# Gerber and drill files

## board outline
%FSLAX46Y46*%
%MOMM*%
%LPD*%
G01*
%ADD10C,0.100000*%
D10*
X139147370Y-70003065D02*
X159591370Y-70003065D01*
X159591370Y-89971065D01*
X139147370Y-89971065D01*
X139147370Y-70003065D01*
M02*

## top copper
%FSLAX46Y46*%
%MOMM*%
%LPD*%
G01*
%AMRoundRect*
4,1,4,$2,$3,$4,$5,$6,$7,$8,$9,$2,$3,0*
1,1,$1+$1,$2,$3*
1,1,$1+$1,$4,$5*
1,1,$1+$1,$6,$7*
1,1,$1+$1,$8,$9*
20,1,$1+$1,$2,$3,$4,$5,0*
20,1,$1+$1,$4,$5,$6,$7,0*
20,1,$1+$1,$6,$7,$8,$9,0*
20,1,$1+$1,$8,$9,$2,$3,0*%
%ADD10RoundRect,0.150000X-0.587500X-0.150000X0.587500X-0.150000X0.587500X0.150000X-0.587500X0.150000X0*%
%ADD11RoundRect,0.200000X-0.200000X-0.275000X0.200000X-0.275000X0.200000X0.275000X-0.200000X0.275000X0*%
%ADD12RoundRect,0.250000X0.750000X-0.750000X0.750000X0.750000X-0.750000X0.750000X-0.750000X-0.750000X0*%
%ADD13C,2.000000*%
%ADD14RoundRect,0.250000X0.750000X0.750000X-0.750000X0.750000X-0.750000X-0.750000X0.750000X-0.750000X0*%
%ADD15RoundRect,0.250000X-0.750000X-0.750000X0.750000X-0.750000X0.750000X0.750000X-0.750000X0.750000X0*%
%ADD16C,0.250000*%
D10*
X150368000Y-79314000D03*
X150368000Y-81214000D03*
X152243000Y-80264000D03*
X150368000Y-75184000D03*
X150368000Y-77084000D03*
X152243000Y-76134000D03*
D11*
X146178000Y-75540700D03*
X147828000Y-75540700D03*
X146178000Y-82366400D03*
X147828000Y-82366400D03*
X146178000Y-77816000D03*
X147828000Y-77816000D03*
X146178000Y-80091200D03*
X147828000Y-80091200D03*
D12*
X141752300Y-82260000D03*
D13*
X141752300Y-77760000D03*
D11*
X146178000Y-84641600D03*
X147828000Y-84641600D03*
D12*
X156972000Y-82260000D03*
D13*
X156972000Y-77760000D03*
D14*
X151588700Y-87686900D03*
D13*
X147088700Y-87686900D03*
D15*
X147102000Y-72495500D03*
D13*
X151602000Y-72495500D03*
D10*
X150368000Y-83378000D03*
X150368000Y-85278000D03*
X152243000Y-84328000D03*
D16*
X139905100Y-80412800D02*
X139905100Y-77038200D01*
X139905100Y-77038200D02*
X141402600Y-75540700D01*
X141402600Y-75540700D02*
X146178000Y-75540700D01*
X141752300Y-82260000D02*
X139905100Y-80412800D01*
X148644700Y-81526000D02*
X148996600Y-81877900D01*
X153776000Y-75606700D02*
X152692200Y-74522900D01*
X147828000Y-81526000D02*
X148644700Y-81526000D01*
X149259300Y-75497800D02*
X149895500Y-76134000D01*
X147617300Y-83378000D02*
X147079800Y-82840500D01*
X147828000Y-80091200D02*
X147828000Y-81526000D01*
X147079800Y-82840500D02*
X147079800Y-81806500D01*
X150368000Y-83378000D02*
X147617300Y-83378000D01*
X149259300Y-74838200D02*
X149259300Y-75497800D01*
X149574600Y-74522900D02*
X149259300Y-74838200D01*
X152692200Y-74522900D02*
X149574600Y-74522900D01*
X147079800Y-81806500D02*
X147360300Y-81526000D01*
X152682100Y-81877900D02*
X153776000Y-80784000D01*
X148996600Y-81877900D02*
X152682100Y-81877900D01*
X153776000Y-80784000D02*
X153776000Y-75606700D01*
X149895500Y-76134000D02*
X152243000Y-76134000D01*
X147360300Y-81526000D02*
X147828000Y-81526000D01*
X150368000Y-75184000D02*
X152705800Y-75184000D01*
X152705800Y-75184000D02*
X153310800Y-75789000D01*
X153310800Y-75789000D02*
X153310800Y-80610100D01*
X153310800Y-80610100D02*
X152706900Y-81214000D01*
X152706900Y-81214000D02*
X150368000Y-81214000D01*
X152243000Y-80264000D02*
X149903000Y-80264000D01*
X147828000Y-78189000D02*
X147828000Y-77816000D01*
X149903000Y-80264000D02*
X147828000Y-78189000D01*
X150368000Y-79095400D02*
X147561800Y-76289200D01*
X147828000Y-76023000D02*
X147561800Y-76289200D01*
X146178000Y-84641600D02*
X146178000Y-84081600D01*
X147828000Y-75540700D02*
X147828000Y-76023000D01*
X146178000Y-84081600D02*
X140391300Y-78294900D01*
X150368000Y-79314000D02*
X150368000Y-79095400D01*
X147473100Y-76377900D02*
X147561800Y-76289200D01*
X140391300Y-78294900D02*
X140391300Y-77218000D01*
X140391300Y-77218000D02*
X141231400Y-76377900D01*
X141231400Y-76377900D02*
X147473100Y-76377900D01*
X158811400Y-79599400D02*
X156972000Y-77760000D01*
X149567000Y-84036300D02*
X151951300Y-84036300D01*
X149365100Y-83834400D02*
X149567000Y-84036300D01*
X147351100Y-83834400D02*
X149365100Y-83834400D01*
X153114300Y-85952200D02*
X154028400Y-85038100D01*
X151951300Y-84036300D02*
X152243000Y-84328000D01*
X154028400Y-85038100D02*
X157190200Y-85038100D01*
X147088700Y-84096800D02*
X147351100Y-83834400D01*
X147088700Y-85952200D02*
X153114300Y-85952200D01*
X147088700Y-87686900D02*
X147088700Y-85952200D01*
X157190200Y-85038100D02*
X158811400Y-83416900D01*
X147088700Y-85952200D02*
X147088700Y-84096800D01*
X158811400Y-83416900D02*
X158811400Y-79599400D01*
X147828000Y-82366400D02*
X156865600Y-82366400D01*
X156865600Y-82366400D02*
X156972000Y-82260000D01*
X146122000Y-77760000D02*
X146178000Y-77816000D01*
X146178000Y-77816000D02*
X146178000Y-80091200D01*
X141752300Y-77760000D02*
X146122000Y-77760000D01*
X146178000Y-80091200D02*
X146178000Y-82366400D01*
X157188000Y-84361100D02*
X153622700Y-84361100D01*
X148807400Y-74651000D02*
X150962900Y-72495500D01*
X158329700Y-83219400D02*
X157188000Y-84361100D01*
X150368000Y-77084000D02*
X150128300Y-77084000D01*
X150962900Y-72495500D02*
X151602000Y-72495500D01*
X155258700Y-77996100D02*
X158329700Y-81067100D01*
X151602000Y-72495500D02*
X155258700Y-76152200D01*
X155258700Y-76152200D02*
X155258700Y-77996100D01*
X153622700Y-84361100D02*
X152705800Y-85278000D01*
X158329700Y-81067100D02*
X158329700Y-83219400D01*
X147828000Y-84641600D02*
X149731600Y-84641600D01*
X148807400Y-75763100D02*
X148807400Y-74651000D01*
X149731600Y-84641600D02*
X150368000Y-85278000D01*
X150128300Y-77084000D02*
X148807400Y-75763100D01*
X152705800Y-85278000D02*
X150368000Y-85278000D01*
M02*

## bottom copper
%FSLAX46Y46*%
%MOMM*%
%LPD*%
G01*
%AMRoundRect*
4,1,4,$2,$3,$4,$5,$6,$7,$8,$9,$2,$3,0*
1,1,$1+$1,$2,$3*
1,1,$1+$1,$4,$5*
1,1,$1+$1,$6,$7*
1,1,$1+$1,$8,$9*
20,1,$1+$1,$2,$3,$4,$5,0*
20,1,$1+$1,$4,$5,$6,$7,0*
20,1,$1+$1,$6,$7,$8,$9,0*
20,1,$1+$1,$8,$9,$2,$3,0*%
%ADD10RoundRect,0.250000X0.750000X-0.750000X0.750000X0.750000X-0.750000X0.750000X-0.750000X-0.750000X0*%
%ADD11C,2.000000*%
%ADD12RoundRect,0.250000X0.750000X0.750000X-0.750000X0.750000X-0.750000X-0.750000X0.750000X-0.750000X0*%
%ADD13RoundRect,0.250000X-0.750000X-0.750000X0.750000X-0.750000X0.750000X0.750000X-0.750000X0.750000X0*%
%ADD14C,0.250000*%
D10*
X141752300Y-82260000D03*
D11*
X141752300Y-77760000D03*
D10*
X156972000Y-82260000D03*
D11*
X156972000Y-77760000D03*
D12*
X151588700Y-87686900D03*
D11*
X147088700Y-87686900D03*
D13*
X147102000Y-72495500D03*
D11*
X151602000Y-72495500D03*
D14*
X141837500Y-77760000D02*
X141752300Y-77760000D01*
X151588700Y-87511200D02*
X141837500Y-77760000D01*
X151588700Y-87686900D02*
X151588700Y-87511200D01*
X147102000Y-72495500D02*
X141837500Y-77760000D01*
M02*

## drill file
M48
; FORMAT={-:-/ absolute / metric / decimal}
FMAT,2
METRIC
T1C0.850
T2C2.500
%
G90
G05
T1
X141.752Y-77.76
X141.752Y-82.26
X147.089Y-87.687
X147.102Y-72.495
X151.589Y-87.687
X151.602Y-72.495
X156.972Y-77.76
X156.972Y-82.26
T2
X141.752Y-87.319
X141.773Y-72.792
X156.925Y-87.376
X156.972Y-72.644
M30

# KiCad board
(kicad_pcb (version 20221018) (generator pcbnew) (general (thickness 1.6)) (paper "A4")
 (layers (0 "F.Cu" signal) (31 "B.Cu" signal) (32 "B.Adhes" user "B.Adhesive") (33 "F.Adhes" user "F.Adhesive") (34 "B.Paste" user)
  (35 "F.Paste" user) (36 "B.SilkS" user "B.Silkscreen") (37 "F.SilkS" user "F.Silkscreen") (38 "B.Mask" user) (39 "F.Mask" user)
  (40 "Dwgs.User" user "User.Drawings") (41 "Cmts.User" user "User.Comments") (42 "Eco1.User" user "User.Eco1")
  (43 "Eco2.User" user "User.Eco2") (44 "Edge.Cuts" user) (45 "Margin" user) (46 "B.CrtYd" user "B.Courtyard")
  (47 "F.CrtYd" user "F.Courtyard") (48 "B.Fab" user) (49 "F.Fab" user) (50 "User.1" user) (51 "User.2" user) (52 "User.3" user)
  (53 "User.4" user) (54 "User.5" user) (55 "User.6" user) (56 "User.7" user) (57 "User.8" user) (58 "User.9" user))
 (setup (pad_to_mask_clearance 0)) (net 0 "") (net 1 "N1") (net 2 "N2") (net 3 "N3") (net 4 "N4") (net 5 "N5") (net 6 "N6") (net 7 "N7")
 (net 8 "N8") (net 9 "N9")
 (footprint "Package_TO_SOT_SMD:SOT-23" (layer "F.Cu") (at 151.3055 80.264)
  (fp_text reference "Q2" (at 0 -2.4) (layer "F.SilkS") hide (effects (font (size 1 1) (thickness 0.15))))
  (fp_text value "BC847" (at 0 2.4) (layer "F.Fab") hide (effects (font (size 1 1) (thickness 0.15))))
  (pad "1" smd roundrect (at -0.9375 -0.95) (size 1.475 0.6) (layers "F.Cu" "F.Paste" "F.Mask") (roundrect_rratio 0.25) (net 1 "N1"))
  (pad "2" smd roundrect (at -0.9375 0.95) (size 1.475 0.6) (layers "F.Cu" "F.Paste" "F.Mask") (roundrect_rratio 0.25) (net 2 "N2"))
  (pad "3" smd roundrect (at 0.9375 0) (size 1.475 0.6) (layers "F.Cu" "F.Paste" "F.Mask") (roundrect_rratio 0.25) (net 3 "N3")))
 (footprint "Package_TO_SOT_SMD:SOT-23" (layer "F.Cu") (at 151.3055 76.134)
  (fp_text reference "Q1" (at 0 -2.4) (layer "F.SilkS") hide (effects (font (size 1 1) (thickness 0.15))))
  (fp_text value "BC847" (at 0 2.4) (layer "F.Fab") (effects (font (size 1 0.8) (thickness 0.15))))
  (pad "1" smd roundrect (at -0.9375 -0.95) (size 1.475 0.6) (layers "F.Cu" "F.Paste" "F.Mask") (roundrect_rratio 0.25) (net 2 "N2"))
  (pad "2" smd roundrect (at -0.9375 0.95) (size 1.475 0.6) (layers "F.Cu" "F.Paste" "F.Mask") (roundrect_rratio 0.25) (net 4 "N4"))
  (pad "3" smd roundrect (at 0.9375 0) (size 1.475 0.6) (layers "F.Cu" "F.Paste" "F.Mask") (roundrect_rratio 0.25) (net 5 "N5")))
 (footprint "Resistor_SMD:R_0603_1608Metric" (layer "F.Cu") (at 147.003 75.5407)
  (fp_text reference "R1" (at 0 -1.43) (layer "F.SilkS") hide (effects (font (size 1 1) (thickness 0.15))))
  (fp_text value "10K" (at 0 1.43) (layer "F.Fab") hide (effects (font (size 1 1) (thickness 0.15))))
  (pad "1" smd roundrect (at -0.825 0) (size 0.8 0.95) (layers "F.Cu" "F.Paste" "F.Mask") (roundrect_rratio 0.25) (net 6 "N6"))
  (pad "2" smd roundrect (at 0.825 0) (size 0.8 0.95) (layers "F.Cu" "F.Paste" "F.Mask") (roundrect_rratio 0.25) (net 1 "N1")))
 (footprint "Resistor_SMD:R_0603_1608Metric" (layer "F.Cu") (at 147.003 82.3664)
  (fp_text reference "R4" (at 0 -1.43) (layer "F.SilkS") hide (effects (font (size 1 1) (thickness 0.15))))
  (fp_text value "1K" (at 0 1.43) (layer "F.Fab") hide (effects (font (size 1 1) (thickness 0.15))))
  (pad "1" smd roundrect (at -0.825 0) (size 0.8 0.95) (layers "F.Cu" "F.Paste" "F.Mask") (roundrect_rratio 0.25) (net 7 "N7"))
  (pad "2" smd roundrect (at 0.825 0) (size 0.8 0.95) (layers "F.Cu" "F.Paste" "F.Mask") (roundrect_rratio 0.25) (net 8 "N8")))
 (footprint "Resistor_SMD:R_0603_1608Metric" (layer "F.Cu") (at 147.003 77.816)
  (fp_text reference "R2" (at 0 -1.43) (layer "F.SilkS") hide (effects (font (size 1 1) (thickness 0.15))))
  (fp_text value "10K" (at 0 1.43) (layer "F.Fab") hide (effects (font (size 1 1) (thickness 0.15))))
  (pad "1" smd roundrect (at -0.825 0) (size 0.8 0.95) (layers "F.Cu" "F.Paste" "F.Mask") (roundrect_rratio 0.25) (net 7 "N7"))
  (pad "2" smd roundrect (at 0.825 0) (size 0.8 0.95) (layers "F.Cu" "F.Paste" "F.Mask") (roundrect_rratio 0.25) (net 3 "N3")))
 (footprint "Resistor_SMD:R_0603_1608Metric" (layer "F.Cu") (at 147.003 80.0912)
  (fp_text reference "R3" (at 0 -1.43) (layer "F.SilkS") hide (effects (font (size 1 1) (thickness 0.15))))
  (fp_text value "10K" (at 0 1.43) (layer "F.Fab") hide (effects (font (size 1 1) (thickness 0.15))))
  (pad "1" smd roundrect (at -0.825 0) (size 0.8 0.95) (layers "F.Cu" "F.Paste" "F.Mask") (roundrect_rratio 0.25) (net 7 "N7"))
  (pad "2" smd roundrect (at 0.825 0) (size 0.8 0.95) (layers "F.Cu" "F.Paste" "F.Mask") (roundrect_rratio 0.25) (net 5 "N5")))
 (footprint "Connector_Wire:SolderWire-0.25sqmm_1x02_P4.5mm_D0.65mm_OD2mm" (layer "F.Cu") (at 141.7523 82.26 90)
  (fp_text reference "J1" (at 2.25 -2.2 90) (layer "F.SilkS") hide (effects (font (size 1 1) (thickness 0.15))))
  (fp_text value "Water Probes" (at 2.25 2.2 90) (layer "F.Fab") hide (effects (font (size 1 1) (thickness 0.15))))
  (pad "1" thru_hole roundrect (at 0 0 90) (size 2 2) (drill 0.85) (layers "*.Cu" "*.Mask") (roundrect_rratio 0.125) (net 6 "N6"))
  (pad "2" thru_hole circle (at 4.5 0 90) (size 2 2) (drill 0.85) (layers "*.Cu" "*.Mask") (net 7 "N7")))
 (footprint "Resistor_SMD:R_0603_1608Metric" (layer "F.Cu") (at 147.003 84.6416)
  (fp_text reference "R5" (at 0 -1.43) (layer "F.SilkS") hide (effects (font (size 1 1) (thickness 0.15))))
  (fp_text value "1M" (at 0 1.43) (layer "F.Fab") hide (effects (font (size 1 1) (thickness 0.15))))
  (pad "1" smd roundrect (at -0.825 0) (size 0.8 0.95) (layers "F.Cu" "F.Paste" "F.Mask") (roundrect_rratio 0.25) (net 1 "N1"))
  (pad "2" smd roundrect (at 0.825 0) (size 0.8 0.95) (layers "F.Cu" "F.Paste" "F.Mask") (roundrect_rratio 0.25) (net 4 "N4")))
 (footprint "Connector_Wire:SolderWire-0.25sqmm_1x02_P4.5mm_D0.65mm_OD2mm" (layer "F.Cu") (at 156.972 82.26 90)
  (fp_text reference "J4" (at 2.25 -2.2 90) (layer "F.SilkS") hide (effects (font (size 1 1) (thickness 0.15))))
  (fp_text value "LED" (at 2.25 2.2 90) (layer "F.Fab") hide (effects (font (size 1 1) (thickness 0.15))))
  (pad "1" thru_hole roundrect (at 0 0 90) (size 2 2) (drill 0.85) (layers "*.Cu" "*.Mask") (roundrect_rratio 0.125) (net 8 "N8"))
  (pad "2" thru_hole circle (at 4.5 0 90) (size 2 2) (drill 0.85) (layers "*.Cu" "*.Mask") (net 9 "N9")))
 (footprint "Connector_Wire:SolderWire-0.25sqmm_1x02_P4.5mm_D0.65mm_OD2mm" (layer "F.Cu") (at 151.5887 87.6869 180)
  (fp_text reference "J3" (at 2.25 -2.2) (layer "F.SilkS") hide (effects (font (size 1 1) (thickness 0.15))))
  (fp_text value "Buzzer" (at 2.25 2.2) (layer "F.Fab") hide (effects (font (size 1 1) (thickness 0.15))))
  (pad "1" thru_hole roundrect (at 0 0 180) (size 2 2) (drill 0.85) (layers "*.Cu" "*.Mask") (roundrect_rratio 0.125) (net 7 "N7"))
  (pad "2" thru_hole circle (at 4.5 0 180) (size 2 2) (drill 0.85) (layers "*.Cu" "*.Mask") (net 9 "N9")))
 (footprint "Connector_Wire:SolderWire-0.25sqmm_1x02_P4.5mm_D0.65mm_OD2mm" (layer "F.Cu") (at 147.102 72.4955)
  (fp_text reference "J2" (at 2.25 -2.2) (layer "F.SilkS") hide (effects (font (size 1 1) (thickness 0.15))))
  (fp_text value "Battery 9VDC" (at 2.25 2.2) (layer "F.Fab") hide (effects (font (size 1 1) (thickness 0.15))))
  (pad "1" thru_hole roundrect (at 0 0) (size 2 2) (drill 0.85) (layers "*.Cu" "*.Mask") (roundrect_rratio 0.125) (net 7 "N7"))
  (pad "2" thru_hole circle (at 4.5 0) (size 2 2) (drill 0.85) (layers "*.Cu" "*.Mask") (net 4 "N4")))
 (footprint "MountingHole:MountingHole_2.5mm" (layer "F.Cu") (at 156.925 87.376)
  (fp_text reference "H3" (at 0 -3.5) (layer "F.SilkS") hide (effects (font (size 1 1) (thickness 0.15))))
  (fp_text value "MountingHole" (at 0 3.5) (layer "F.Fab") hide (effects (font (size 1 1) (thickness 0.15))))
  (pad "" np_thru_hole circle (at 0 0) (size 2.5 2.5) (drill 2.5) (layers "*.Cu" "*.Mask")))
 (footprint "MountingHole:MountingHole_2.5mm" (layer "F.Cu") (at 141.7523 87.3191)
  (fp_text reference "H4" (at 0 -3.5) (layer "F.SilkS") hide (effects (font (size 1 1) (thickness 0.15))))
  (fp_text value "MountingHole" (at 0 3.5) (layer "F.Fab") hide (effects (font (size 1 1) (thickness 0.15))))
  (pad "" np_thru_hole circle (at 0 0) (size 2.5 2.5) (drill 2.5) (layers "*.Cu" "*.Mask")))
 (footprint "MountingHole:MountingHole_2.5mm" (layer "F.Cu") (at 141.7726 72.7925)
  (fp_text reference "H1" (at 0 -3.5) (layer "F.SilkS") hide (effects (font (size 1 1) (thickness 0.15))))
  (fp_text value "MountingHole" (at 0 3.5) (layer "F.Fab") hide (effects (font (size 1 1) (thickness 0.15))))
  (pad "" np_thru_hole circle (at 0 0) (size 2.5 2.5) (drill 2.5) (layers "*.Cu" "*.Mask")))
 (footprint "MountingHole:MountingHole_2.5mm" (layer "F.Cu") (at 156.972 72.644)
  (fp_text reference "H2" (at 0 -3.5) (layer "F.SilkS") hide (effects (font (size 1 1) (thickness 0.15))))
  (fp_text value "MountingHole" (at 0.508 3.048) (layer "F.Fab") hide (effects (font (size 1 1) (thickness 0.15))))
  (pad "" np_thru_hole circle (at 0 0) (size 2.5 2.5) (drill 2.5) (layers "*.Cu" "*.Mask")))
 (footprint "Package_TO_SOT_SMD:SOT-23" (layer "F.Cu") (at 151.3055 84.328)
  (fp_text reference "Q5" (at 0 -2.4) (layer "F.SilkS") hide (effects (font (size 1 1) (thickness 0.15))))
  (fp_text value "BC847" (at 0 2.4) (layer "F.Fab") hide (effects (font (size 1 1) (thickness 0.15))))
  (pad "1" smd roundrect (at -0.9375 -0.95) (size 1.475 0.6) (layers "F.Cu" "F.Paste" "F.Mask") (roundrect_rratio 0.25) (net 5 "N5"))
  (pad "2" smd roundrect (at -0.9375 0.95) (size 1.475 0.6) (layers "F.Cu" "F.Paste" "F.Mask") (roundrect_rratio 0.25) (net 4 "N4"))
  (pad "3" smd roundrect (at 0.9375 0) (size 1.475 0.6) (layers "F.Cu" "F.Paste" "F.Mask") (roundrect_rratio 0.25) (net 9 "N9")))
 (gr_rect (start 139.14737 70.003065) (end 159.59137 89.971065) (stroke (width 0.1) (type default)) (fill none) (layer "Edge.Cuts"))
 (segment (start 139.9051 80.4128) (end 139.9051 77.0382) (width 0.25) (layer "F.Cu") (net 6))
 (segment (start 139.9051 77.0382) (end 141.4026 75.5407) (width 0.25) (layer "F.Cu") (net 6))
 (segment (start 141.4026 75.5407) (end 146.178 75.5407) (width 0.25) (layer "F.Cu") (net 6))
 (segment (start 141.7523 82.26) (end 139.9051 80.4128) (width 0.25) (layer "F.Cu") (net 6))
 (segment (start 148.6447 81.526) (end 148.9966 81.8779) (width 0.25) (layer "F.Cu") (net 5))
 (segment (start 153.776 75.6067) (end 152.6922 74.5229) (width 0.25) (layer "F.Cu") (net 5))
 (segment (start 147.828 81.526) (end 148.6447 81.526) (width 0.25) (layer "F.Cu") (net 5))
 (segment (start 149.2593 75.4978) (end 149.8955 76.134) (width 0.25) (layer "F.Cu") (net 5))
 (segment (start 147.6173 83.378) (end 147.0798 82.8405) (width 0.25) (layer "F.Cu") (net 5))
 (segment (start 147.828 80.0912) (end 147.828 81.526) (width 0.25) (layer "F.Cu") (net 5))
 (segment (start 147.0798 82.8405) (end 147.0798 81.8065) (width 0.25) (layer "F.Cu") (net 5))
 (segment (start 150.368 83.378) (end 147.6173 83.378) (width 0.25) (layer "F.Cu") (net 5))
 (segment (start 149.2593 74.8382) (end 149.2593 75.4978) (width 0.25) (layer "F.Cu") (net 5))
 (segment (start 149.5746 74.5229) (end 149.2593 74.8382) (width 0.25) (layer "F.Cu") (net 5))
 (segment (start 152.6922 74.5229) (end 149.5746 74.5229) (width 0.25) (layer "F.Cu") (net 5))
 (segment (start 147.0798 81.8065) (end 147.3603 81.526) (width 0.25) (layer "F.Cu") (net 5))
 (segment (start 152.6821 81.8779) (end 153.776 80.784) (width 0.25) (layer "F.Cu") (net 5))
 (segment (start 148.9966 81.8779) (end 152.6821 81.8779) (width 0.25) (layer "F.Cu") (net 5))
 (segment (start 153.776 80.784) (end 153.776 75.6067) (width 0.25) (layer "F.Cu") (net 5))
 (segment (start 149.8955 76.134) (end 152.243 76.134) (width 0.25) (layer "F.Cu") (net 5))
 (segment (start 147.3603 81.526) (end 147.828 81.526) (width 0.25) (layer "F.Cu") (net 5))
 (segment (start 150.368 75.184) (end 152.7058 75.184) (width 0.25) (layer "F.Cu") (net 2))
 (segment (start 152.7058 75.184) (end 153.3108 75.789) (width 0.25) (layer "F.Cu") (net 2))
 (segment (start 153.3108 75.789) (end 153.3108 80.6101) (width 0.25) (layer "F.Cu") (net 2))
 (segment (start 153.3108 80.6101) (end 152.7069 81.214) (width 0.25) (layer "F.Cu") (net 2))
 (segment (start 152.7069 81.214) (end 150.368 81.214) (width 0.25) (layer "F.Cu") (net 2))
 (segment (start 152.243 80.264) (end 149.903 80.264) (width 0.25) (layer "F.Cu") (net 3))
 (segment (start 147.828 78.189) (end 147.828 77.816) (width 0.25) (layer "F.Cu") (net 3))
 (segment (start 149.903 80.264) (end 147.828 78.189) (width 0.25) (layer "F.Cu") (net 3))
 (segment (start 150.368 79.0954) (end 147.5618 76.2892) (width 0.25) (layer "F.Cu") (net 1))
 (segment (start 147.828 76.023) (end 147.5618 76.2892) (width 0.25) (layer "F.Cu") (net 1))
 (segment (start 146.178 84.6416) (end 146.178 84.0816) (width 0.25) (layer "F.Cu") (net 1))
 (segment (start 147.828 75.5407) (end 147.828 76.023) (width 0.25) (layer "F.Cu") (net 1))
 (segment (start 146.178 84.0816) (end 140.3913 78.2949) (width 0.25) (layer "F.Cu") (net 1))
 (segment (start 150.368 79.314) (end 150.368 79.0954) (width 0.25) (layer "F.Cu") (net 1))
 (segment (start 147.4731 76.3779) (end 147.5618 76.2892) (width 0.25) (layer "F.Cu") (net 1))
 (segment (start 140.3913 78.2949) (end 140.3913 77.218) (width 0.25) (layer "F.Cu") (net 1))
 (segment (start 140.3913 77.218) (end 141.2314 76.3779) (width 0.25) (layer "F.Cu") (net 1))
 (segment (start 141.2314 76.3779) (end 147.4731 76.3779) (width 0.25) (layer "F.Cu") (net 1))
 (segment (start 158.8114 79.5994) (end 156.972 77.76) (width 0.25) (layer "F.Cu") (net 9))
 (segment (start 149.567 84.0363) (end 151.9513 84.0363) (width 0.25) (layer "F.Cu") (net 9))
 (segment (start 149.3651 83.8344) (end 149.567 84.0363) (width 0.25) (layer "F.Cu") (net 9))
 (segment (start 147.3511 83.8344) (end 149.3651 83.8344) (width 0.25) (layer "F.Cu") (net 9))
 (segment (start 153.1143 85.9522) (end 154.0284 85.0381) (width 0.25) (layer "F.Cu") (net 9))
 (segment (start 151.9513 84.0363) (end 152.243 84.328) (width 0.25) (layer "F.Cu") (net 9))
 (segment (start 154.0284 85.0381) (end 157.1902 85.0381) (width 0.25) (layer "F.Cu") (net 9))
 (segment (start 147.0887 84.0968) (end 147.3511 83.8344) (width 0.25) (layer "F.Cu") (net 9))
 (segment (start 147.0887 85.9522) (end 153.1143 85.9522) (width 0.25) (layer "F.Cu") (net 9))
 (segment (start 147.0887 87.6869) (end 147.0887 85.9522) (width 0.25) (layer "F.Cu") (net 9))
 (segment (start 157.1902 85.0381) (end 158.8114 83.4169) (width 0.25) (layer "F.Cu") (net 9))
 (segment (start 147.0887 85.9522) (end 147.0887 84.0968) (width 0.25) (layer "F.Cu") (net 9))
 (segment (start 158.8114 83.4169) (end 158.8114 79.5994) (width 0.25) (layer "F.Cu") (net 9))
 (segment (start 147.828 82.3664) (end 156.8656 82.3664) (width 0.25) (layer "F.Cu") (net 8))
 (segment (start 156.8656 82.3664) (end 156.972 82.26) (width 0.25) (layer "F.Cu") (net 8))
 (segment (start 146.122 77.76) (end 146.178 77.816) (width 0.25) (layer "F.Cu") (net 7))
 (segment (start 146.178 77.816) (end 146.178 80.0912) (width 0.25) (layer "F.Cu") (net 7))
 (segment (start 141.7523 77.76) (end 146.122 77.76) (width 0.25) (layer "F.Cu") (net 7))
 (segment (start 146.178 80.0912) (end 146.178 82.3664) (width 0.25) (layer "F.Cu") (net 7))
 (segment (start 141.8375 77.76) (end 141.7523 77.76) (width 0.25) (layer "B.Cu") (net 7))
 (segment (start 151.5887 87.5112) (end 141.8375 77.76) (width 0.25) (layer "B.Cu") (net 7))
 (segment (start 151.5887 87.6869) (end 151.5887 87.5112) (width 0.25) (layer "B.Cu") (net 7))
 (segment (start 147.102 72.4955) (end 141.8375 77.76) (width 0.25) (layer "B.Cu") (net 7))
 (segment (start 157.188 84.3611) (end 153.6227 84.3611) (width 0.25) (layer "F.Cu") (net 4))
 (segment (start 148.8074 74.651) (end 150.9629 72.4955) (width 0.25) (layer "F.Cu") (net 4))
 (segment (start 158.3297 83.2194) (end 157.188 84.3611) (width 0.25) (layer "F.Cu") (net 4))
 (segment (start 150.368 77.084) (end 150.1283 77.084) (width 0.25) (layer "F.Cu") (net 4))
 (segment (start 150.9629 72.4955) (end 151.602 72.4955) (width 0.25) (layer "F.Cu") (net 4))
 (segment (start 155.2587 77.9961) (end 158.3297 81.0671) (width 0.25) (layer "F.Cu") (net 4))
 (segment (start 151.602 72.4955) (end 155.2587 76.1522) (width 0.25) (layer "F.Cu") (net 4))
 (segment (start 155.2587 76.1522) (end 155.2587 77.9961) (width 0.25) (layer "F.Cu") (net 4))
 (segment (start 153.6227 84.3611) (end 152.7058 85.278) (width 0.25) (layer "F.Cu") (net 4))
 (segment (start 158.3297 81.0671) (end 158.3297 83.2194) (width 0.25) (layer "F.Cu") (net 4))
 (segment (start 147.828 84.6416) (end 149.7316 84.6416) (width 0.25) (layer "F.Cu") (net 4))
 (segment (start 148.8074 75.7631) (end 148.8074 74.651) (width 0.25) (layer "F.Cu") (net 4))
 (segment (start 149.7316 84.6416) (end 150.368 85.278) (width 0.25) (layer "F.Cu") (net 4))
 (segment (start 150.1283 77.084) (end 148.8074 75.7631) (width 0.25) (layer "F.Cu") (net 4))
 (segment (start 152.7058 85.278) (end 150.368 85.278) (width 0.25) (layer "F.Cu") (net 4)))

